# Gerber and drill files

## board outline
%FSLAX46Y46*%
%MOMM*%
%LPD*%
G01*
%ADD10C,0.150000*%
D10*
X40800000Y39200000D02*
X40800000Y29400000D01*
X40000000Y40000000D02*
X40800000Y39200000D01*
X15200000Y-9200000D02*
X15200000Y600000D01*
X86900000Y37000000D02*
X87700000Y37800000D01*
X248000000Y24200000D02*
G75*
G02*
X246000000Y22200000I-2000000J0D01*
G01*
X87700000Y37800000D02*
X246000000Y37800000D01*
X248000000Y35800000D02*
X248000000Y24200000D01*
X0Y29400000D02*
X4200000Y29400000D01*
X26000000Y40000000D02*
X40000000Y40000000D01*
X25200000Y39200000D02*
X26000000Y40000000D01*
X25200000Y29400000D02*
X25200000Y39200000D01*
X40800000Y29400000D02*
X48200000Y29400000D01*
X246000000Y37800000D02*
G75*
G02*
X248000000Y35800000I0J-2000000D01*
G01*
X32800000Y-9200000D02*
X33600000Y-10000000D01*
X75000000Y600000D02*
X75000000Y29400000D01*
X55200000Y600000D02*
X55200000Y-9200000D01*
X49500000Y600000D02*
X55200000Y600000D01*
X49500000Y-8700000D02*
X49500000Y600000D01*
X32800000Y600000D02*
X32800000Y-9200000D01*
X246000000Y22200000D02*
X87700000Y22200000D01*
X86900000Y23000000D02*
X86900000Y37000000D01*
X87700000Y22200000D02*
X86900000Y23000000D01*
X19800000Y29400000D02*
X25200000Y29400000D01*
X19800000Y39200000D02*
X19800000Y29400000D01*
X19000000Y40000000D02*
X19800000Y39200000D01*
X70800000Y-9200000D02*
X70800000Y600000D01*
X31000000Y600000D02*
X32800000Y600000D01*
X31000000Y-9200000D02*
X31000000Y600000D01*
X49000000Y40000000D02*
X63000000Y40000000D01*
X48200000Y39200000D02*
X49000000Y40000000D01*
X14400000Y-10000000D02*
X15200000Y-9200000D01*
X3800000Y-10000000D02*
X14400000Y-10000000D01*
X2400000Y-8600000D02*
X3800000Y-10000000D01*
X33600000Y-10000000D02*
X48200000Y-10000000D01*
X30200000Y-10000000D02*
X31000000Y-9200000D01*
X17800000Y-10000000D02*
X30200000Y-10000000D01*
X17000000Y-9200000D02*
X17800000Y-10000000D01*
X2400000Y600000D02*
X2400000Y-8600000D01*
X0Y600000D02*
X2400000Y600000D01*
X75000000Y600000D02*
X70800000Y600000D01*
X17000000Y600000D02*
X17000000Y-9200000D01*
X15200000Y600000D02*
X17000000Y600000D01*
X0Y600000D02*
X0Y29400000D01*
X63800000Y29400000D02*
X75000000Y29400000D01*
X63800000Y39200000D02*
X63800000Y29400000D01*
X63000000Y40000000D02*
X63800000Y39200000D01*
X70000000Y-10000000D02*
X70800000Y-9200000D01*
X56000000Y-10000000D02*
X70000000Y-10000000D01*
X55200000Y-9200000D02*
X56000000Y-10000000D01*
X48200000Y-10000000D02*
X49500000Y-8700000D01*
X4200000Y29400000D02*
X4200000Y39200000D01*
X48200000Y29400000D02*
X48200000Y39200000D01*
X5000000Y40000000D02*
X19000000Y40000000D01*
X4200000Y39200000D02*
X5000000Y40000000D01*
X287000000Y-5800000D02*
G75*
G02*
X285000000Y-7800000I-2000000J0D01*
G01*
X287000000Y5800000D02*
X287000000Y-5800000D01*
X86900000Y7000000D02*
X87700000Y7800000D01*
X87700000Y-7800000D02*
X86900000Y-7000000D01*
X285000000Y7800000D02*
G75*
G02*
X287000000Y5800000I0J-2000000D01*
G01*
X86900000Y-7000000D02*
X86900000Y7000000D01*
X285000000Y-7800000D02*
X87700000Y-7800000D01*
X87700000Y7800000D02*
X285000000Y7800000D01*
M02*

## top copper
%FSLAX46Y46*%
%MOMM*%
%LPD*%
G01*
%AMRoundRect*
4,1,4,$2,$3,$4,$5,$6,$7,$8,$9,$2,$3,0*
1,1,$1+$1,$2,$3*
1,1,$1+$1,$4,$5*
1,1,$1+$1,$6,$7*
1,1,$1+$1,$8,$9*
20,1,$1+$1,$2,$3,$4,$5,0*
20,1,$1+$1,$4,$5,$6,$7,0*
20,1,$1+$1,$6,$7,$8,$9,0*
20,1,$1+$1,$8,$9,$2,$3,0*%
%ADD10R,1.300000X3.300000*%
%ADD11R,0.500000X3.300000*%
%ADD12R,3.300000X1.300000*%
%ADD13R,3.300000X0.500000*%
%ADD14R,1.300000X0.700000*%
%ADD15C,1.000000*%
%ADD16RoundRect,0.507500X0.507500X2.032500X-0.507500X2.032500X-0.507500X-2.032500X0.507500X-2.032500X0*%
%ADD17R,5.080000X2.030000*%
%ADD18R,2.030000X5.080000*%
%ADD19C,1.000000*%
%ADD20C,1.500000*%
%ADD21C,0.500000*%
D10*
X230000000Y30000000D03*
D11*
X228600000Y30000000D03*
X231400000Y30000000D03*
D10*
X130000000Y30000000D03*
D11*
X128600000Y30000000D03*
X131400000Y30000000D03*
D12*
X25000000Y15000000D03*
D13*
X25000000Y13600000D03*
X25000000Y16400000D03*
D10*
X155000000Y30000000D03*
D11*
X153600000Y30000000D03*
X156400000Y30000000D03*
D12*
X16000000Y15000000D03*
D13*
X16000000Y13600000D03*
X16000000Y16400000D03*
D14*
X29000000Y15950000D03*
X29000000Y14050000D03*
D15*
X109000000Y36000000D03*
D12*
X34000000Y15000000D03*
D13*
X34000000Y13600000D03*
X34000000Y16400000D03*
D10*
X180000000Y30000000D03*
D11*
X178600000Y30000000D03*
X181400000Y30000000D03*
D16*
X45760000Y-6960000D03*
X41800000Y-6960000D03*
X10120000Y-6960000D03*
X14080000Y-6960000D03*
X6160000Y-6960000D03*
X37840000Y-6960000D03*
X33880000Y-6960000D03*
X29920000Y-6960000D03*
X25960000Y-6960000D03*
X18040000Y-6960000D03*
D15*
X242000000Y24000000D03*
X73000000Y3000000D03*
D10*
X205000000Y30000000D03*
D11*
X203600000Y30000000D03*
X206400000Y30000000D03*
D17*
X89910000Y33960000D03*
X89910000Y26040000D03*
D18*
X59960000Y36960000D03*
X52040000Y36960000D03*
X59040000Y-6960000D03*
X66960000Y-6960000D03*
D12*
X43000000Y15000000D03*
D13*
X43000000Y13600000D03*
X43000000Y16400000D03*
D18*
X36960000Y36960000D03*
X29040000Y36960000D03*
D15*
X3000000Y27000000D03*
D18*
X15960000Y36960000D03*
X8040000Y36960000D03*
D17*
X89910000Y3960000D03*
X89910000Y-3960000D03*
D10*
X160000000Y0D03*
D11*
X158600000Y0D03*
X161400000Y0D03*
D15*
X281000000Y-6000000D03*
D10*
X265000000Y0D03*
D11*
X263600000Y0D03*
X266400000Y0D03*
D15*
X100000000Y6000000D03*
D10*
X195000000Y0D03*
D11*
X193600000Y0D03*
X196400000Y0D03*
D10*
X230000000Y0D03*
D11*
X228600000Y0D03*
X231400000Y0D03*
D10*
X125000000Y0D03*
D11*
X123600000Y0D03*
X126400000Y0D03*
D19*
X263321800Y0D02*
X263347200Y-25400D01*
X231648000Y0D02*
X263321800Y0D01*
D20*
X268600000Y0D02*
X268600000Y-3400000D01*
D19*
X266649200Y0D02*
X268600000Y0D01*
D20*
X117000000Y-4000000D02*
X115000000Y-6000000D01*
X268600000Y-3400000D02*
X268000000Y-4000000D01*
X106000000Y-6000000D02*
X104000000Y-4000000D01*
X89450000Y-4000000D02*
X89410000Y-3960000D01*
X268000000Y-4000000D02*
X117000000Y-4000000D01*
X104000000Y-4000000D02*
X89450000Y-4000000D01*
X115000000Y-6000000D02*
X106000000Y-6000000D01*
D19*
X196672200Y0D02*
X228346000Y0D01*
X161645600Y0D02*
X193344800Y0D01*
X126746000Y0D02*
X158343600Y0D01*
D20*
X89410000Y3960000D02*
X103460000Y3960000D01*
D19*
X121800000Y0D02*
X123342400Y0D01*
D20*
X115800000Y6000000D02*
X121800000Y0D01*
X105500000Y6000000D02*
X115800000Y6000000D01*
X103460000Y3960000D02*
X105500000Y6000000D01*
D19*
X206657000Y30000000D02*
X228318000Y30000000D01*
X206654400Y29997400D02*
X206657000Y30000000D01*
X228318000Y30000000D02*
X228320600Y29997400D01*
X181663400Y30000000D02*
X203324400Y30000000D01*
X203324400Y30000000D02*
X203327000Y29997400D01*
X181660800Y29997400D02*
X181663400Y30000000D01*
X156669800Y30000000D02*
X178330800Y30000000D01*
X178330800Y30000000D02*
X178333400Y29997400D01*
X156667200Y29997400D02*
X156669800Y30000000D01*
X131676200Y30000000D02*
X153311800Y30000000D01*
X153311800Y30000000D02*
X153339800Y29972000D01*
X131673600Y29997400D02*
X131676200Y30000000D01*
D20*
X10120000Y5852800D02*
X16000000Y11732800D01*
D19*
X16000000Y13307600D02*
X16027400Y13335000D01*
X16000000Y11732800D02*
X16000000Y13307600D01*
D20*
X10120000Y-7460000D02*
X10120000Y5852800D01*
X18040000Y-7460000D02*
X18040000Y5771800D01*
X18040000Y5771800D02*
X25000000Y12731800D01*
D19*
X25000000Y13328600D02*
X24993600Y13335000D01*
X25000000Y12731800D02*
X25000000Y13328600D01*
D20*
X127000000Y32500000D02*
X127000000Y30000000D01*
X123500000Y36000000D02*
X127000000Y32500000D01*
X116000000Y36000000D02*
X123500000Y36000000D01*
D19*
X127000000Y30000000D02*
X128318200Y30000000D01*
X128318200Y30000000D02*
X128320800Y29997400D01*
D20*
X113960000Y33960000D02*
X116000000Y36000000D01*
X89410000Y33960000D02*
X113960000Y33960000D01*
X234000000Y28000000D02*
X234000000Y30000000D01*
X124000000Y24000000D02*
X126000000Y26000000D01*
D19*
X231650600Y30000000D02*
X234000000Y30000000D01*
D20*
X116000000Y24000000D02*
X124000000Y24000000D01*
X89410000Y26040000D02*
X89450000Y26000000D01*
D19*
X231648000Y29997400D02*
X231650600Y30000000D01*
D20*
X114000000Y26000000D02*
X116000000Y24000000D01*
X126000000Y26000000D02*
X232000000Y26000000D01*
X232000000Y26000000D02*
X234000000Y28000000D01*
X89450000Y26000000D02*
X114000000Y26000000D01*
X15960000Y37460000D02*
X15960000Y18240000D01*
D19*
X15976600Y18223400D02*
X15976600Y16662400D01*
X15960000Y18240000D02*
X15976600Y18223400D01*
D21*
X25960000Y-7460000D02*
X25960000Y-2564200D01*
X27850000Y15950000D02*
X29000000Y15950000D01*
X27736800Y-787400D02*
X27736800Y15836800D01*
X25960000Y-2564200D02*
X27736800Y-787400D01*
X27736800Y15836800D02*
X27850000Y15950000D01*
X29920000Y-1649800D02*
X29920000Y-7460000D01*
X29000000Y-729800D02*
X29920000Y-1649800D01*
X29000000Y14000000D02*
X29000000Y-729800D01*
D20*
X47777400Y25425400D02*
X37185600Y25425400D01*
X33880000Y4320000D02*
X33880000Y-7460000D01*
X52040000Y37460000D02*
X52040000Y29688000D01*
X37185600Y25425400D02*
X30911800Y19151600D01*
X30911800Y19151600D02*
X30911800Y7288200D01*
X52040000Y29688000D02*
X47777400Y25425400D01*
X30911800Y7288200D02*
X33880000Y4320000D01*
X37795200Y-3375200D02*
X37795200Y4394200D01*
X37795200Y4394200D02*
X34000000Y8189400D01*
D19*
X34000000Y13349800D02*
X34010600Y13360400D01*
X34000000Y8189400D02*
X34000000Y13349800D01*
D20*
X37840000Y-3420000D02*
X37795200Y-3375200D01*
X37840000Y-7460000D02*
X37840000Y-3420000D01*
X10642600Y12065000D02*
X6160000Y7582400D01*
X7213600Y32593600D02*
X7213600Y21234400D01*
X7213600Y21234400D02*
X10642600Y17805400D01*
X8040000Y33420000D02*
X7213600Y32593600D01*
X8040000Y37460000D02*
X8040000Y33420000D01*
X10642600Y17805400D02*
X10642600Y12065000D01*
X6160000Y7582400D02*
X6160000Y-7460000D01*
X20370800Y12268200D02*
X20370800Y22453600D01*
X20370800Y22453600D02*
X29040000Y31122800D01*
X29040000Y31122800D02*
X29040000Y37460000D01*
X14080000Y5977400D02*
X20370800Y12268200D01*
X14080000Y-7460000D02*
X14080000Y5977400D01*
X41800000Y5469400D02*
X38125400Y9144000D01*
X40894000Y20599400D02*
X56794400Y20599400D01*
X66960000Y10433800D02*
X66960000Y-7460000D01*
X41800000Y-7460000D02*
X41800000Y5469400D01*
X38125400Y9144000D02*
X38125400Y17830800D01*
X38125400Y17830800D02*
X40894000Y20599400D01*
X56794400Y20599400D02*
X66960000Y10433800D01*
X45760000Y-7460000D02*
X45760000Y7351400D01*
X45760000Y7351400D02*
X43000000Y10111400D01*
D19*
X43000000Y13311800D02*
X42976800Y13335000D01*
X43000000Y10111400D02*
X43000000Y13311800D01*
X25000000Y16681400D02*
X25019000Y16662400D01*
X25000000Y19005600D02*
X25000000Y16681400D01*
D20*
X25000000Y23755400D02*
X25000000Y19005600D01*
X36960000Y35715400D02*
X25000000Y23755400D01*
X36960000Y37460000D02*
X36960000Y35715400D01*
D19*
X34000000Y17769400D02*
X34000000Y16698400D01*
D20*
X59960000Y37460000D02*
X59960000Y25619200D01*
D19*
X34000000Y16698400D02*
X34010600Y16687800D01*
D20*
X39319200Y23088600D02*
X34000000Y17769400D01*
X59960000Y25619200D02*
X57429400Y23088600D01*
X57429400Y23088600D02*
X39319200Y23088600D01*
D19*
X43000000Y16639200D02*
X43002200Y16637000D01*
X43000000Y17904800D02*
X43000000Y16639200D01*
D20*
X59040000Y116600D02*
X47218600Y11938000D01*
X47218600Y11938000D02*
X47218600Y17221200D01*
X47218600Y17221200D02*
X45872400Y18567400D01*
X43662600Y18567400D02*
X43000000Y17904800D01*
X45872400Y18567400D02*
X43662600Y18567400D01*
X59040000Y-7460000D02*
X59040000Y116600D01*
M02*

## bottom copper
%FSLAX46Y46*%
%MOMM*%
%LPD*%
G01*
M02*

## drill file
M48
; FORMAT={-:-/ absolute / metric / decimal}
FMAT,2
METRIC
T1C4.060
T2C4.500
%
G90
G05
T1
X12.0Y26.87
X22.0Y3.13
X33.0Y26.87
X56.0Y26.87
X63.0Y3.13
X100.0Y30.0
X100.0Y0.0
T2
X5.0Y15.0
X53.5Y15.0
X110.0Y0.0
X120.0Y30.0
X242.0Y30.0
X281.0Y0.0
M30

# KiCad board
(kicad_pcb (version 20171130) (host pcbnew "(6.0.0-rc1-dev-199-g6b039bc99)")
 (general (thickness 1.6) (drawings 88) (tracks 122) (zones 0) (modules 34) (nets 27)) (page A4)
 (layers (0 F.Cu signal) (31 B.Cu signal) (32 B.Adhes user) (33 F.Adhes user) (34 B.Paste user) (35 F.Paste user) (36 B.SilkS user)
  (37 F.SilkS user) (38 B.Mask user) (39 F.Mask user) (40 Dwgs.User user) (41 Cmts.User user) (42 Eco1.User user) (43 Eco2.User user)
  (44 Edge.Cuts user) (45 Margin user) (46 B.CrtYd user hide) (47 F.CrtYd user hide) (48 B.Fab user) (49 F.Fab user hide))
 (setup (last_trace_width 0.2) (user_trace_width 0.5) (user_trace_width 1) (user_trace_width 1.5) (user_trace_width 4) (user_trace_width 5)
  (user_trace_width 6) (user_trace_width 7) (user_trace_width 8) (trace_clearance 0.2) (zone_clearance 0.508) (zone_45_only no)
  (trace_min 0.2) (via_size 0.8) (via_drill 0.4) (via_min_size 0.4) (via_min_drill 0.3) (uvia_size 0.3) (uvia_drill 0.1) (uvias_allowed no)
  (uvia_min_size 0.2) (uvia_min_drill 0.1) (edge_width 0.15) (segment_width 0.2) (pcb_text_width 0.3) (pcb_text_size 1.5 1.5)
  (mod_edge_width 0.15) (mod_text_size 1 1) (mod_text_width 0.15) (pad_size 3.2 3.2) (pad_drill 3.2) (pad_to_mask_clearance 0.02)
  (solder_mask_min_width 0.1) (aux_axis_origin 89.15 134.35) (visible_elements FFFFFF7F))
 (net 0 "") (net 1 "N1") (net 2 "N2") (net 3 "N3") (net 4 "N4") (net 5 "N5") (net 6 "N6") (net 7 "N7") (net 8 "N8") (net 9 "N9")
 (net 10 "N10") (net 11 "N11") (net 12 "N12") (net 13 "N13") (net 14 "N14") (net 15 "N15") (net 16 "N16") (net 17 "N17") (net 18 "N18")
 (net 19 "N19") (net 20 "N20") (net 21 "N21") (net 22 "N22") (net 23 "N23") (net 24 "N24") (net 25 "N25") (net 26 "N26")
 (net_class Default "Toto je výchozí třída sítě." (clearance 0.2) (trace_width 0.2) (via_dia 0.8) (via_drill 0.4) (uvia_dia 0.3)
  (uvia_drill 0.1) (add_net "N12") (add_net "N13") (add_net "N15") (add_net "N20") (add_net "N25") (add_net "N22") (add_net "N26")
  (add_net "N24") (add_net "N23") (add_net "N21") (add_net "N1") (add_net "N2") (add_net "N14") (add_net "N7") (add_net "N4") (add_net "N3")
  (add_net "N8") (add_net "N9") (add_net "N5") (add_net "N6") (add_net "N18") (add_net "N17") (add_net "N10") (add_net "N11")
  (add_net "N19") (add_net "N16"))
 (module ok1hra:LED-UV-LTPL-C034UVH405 (layer F.Cu) (at 230 -30)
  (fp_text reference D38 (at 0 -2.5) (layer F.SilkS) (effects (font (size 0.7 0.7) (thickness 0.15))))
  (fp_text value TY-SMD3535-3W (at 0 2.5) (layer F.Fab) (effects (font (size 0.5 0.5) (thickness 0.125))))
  (pad 3 smd rect (at 0 0) (size 1.3 3.3) (layers F.Cu F.Paste F.Mask))
  (pad 1 smd rect (at -1.4 0) (size 0.5 3.3) (layers F.Cu F.Paste F.Mask) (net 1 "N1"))
  (pad 2 smd rect (at 1.4 0) (size 0.5 3.3) (layers F.Cu F.Paste F.Mask) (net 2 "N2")))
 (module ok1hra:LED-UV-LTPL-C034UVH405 (layer F.Cu) (at 130 -30)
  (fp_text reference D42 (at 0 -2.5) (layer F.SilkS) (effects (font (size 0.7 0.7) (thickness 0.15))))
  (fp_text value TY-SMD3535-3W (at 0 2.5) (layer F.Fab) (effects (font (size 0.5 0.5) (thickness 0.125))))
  (pad 3 smd rect (at 0 0) (size 1.3 3.3) (layers F.Cu F.Paste F.Mask))
  (pad 1 smd rect (at -1.4 0) (size 0.5 3.3) (layers F.Cu F.Paste F.Mask) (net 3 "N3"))
  (pad 2 smd rect (at 1.4 0) (size 0.5 3.3) (layers F.Cu F.Paste F.Mask) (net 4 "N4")))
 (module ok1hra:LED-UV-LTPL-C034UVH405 (layer F.Cu) (at 25 -15 90)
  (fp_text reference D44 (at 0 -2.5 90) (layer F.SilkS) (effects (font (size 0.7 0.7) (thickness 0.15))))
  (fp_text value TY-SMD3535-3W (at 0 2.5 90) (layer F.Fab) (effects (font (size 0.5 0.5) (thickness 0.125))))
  (pad 3 smd rect (at 0 0 90) (size 1.3 3.3) (layers F.Cu F.Paste F.Mask))
  (pad 1 smd rect (at -1.4 0 90) (size 0.5 3.3) (layers F.Cu F.Paste F.Mask) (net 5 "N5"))
  (pad 2 smd rect (at 1.4 0 90) (size 0.5 3.3) (layers F.Cu F.Paste F.Mask) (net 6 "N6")))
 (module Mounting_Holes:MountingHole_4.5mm (layer F.Cu) (at 242 -30)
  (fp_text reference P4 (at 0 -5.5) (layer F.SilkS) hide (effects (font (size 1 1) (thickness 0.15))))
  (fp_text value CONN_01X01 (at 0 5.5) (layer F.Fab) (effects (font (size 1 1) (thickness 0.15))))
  (pad 1 np_thru_hole circle (at 0 0) (size 4.5 4.5) (drill 4.5) (layers *.Cu *.Mask)))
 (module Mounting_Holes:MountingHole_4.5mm (layer F.Cu) (at 5 -15)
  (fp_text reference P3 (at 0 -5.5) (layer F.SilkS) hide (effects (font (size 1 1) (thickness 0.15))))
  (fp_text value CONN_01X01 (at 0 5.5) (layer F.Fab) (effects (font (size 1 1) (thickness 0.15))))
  (pad 1 np_thru_hole circle (at 0 0) (size 4.5 4.5) (drill 4.5) (layers *.Cu *.Mask)))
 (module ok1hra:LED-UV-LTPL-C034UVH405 (layer F.Cu) (at 155 -30)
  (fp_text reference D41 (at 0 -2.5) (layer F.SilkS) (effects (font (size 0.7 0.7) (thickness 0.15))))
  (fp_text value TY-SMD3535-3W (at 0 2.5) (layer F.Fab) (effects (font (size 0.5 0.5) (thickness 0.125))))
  (pad 3 smd rect (at 0 0) (size 1.3 3.3) (layers F.Cu F.Paste F.Mask))
  (pad 1 smd rect (at -1.4 0) (size 0.5 3.3) (layers F.Cu F.Paste F.Mask) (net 4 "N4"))
  (pad 2 smd rect (at 1.4 0) (size 0.5 3.3) (layers F.Cu F.Paste F.Mask) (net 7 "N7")))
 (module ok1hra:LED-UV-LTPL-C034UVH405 (layer F.Cu) (at 16 -15 90)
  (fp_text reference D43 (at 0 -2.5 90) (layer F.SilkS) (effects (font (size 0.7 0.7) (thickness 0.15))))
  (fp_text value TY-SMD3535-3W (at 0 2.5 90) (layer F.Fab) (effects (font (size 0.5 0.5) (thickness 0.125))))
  (pad 3 smd rect (at 0 0 90) (size 1.3 3.3) (layers F.Cu F.Paste F.Mask))
  (pad 1 smd rect (at -1.4 0 90) (size 0.5 3.3) (layers F.Cu F.Paste F.Mask) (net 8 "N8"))
  (pad 2 smd rect (at 1.4 0 90) (size 0.5 3.3) (layers F.Cu F.Paste F.Mask) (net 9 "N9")))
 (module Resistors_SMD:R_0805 (layer F.Cu) (at 29 -15 270)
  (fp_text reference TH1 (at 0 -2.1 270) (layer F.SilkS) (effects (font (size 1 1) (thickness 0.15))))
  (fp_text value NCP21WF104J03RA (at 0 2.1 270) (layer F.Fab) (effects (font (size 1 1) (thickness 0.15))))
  (pad 1 smd rect (at -0.95 0 270) (size 0.7 1.3) (layers F.Cu F.Paste F.Mask) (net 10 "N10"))
  (pad 2 smd rect (at 0.95 0 270) (size 0.7 1.3) (layers F.Cu F.Paste F.Mask) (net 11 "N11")))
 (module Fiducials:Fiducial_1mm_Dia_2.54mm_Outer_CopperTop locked (layer F.Cu) (at 109 -36)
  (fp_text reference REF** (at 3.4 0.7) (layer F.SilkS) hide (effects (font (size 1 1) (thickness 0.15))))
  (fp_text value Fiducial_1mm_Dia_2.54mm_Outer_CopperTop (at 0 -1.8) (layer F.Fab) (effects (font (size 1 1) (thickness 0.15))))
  (pad ~ smd circle (at 0 0) (size 1 1) (layers F.Cu F.Mask) (solder_mask_margin 0.77) (clearance 0.77)))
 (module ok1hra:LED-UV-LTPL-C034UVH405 (layer F.Cu) (at 34 -15 90)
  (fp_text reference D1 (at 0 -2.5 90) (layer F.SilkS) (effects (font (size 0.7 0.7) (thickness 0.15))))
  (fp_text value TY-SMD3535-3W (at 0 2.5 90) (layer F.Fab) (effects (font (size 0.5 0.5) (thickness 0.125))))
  (pad 3 smd rect (at 0 0 90) (size 1.3 3.3) (layers F.Cu F.Paste F.Mask))
  (pad 1 smd rect (at -1.4 0 90) (size 0.5 3.3) (layers F.Cu F.Paste F.Mask) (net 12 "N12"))
  (pad 2 smd rect (at 1.4 0 90) (size 0.5 3.3) (layers F.Cu F.Paste F.Mask) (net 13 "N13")))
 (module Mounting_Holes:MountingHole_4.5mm (layer F.Cu) (at 53.5 -15)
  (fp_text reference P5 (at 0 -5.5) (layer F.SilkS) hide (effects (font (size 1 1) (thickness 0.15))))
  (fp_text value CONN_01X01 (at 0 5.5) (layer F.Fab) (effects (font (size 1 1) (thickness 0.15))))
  (pad 1 np_thru_hole circle (at 0 0) (size 4.5 4.5) (drill 4.5) (layers *.Cu *.Mask)))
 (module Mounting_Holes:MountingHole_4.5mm (layer F.Cu) (at 120 -30)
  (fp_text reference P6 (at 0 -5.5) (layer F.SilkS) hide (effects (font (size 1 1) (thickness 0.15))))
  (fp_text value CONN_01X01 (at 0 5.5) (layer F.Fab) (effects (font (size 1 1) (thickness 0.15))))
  (pad 1 np_thru_hole circle (at 0 0) (size 4.5 4.5) (drill 4.5) (layers *.Cu *.Mask)))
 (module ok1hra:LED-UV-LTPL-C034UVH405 (layer F.Cu) (at 180 -30)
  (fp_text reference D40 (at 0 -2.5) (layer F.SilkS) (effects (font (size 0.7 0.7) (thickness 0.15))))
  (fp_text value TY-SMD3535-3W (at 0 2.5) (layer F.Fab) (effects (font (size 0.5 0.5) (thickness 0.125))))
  (pad 3 smd rect (at 0 0) (size 1.3 3.3) (layers F.Cu F.Paste F.Mask))
  (pad 1 smd rect (at -1.4 0) (size 0.5 3.3) (layers F.Cu F.Paste F.Mask) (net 7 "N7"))
  (pad 2 smd rect (at 1.4 0) (size 0.5 3.3) (layers F.Cu F.Paste F.Mask) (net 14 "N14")))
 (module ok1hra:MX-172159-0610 (layer F.Cu) (at 22 10 180)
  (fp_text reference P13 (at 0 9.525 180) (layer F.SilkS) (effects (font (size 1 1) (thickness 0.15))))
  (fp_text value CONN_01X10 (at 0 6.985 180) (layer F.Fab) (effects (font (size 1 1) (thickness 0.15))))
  (pad 10 smd roundrect (at -23.76 3.04 180) (size 2.03 5.08) (layers F.Cu F.Mask) (roundrect_rratio 0.25) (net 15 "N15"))
  (pad 9 smd roundrect (at -19.8 3.04 180) (size 2.03 5.08) (layers F.Cu F.Mask) (roundrect_rratio 0.25) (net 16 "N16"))
  (pad 2 smd roundrect (at 11.88 3.04 180) (size 2.03 5.08) (layers F.Cu F.Mask) (roundrect_rratio 0.25) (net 8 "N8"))
  (pad 3 smd roundrect (at 7.92 3.04 180) (size 2.03 5.08) (layers F.Cu F.Mask) (roundrect_rratio 0.25) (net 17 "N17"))
  (pad 1 smd roundrect (at 15.84 3.04 180) (size 2.03 5.08) (layers F.Cu F.Mask) (roundrect_rratio 0.25) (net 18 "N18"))
  (pad 8 smd roundrect (at -15.84 3.04 180) (size 2.03 5.08) (layers F.Cu F.Mask) (roundrect_rratio 0.25) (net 12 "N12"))
  (pad 7 smd roundrect (at -11.88 3.04 180) (size 2.03 5.08) (layers F.Cu F.Mask) (roundrect_rratio 0.25) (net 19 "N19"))
  (pad 6 smd roundrect (at -7.92 3.04 180) (size 2.03 5.08) (layers F.Cu F.Mask) (roundrect_rratio 0.25) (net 11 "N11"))
  (pad 5 smd roundrect (at -3.96 3.04 180) (size 2.03 5.08) (layers F.Cu F.Mask) (roundrect_rratio 0.25) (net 10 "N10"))
  (pad 4 smd roundrect (at 3.96 3.04 180) (size 2.03 5.08) (layers F.Cu F.Mask) (roundrect_rratio 0.25) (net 5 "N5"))
  (pad "" np_thru_hole circle (at 0 13.13 180) (size 4.06 4.06) (drill 4.06) (layers *.Cu *.Mask)))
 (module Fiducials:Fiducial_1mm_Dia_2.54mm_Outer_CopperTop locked (layer F.Cu) (at 242 -24)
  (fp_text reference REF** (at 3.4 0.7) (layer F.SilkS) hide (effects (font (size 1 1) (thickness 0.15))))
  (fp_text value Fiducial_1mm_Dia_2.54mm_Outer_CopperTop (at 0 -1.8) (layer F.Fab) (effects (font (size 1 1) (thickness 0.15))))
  (pad ~ smd circle (at 0 0) (size 1 1) (layers F.Cu F.Mask) (solder_mask_margin 0.77) (clearance 0.77)))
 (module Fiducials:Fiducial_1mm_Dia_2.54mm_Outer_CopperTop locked (layer F.Cu) (at 73 -3)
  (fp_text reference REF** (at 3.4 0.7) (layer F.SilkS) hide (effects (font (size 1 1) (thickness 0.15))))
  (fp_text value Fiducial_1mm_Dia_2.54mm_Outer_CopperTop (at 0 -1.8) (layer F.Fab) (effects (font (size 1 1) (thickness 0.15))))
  (pad ~ smd circle (at 0 0) (size 1 1) (layers F.Cu F.Mask) (solder_mask_margin 0.77) (clearance 0.77)))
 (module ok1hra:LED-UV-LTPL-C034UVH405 (layer F.Cu) (at 205 -30)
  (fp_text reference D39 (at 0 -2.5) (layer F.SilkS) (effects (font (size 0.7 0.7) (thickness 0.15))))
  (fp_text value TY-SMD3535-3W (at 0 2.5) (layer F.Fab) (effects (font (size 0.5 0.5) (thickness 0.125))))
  (pad 3 smd rect (at 0 0) (size 1.3 3.3) (layers F.Cu F.Paste F.Mask))
  (pad 1 smd rect (at -1.4 0) (size 0.5 3.3) (layers F.Cu F.Paste F.Mask) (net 14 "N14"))
  (pad 2 smd rect (at 1.4 0) (size 0.5 3.3) (layers F.Cu F.Paste F.Mask) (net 1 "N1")))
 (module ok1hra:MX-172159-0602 (layer F.Cu) (at 86.87 -30 90)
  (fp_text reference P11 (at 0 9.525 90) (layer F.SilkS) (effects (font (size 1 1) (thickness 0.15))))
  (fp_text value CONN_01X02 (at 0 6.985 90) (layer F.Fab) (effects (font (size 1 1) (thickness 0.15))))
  (pad "" np_thru_hole circle (at 0 13.13 90) (size 4.06 4.06) (drill 4.06) (layers *.Cu *.Mask))
  (pad 1 smd rect (at 3.96 3.04 90) (size 2.03 5.08) (layers F.Cu F.Mask) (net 3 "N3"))
  (pad 2 smd rect (at -3.96 3.04 90) (size 2.03 5.08) (layers F.Cu F.Mask) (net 2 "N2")))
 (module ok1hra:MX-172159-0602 (layer F.Cu) (at 56 -40)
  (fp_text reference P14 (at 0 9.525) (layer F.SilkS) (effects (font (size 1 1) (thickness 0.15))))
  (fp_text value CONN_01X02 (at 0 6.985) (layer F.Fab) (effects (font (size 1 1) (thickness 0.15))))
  (pad "" np_thru_hole circle (at 0 13.13) (size 4.06 4.06) (drill 4.06) (layers *.Cu *.Mask))
  (pad 1 smd rect (at 3.96 3.04) (size 2.03 5.08) (layers F.Cu F.Mask) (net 13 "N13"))
  (pad 2 smd rect (at -3.96 3.04) (size 2.03 5.08) (layers F.Cu F.Mask) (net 19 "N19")))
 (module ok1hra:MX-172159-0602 (layer F.Cu) (at 63 10 180)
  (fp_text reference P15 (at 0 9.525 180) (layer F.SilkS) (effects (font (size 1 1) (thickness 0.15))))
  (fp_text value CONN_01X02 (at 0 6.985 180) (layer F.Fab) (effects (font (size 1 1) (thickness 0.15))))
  (pad "" np_thru_hole circle (at 0 13.13 180) (size 4.06 4.06) (drill 4.06) (layers *.Cu *.Mask))
  (pad 1 smd rect (at 3.96 3.04 180) (size 2.03 5.08) (layers F.Cu F.Mask) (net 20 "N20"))
  (pad 2 smd rect (at -3.96 3.04 180) (size 2.03 5.08) (layers F.Cu F.Mask) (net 16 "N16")))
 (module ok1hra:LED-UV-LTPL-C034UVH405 (layer F.Cu) (at 43 -15 90)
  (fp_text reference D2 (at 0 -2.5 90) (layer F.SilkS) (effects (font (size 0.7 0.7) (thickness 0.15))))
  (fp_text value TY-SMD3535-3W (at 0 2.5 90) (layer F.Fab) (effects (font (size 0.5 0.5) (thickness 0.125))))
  (pad 3 smd rect (at 0 0 90) (size 1.3 3.3) (layers F.Cu F.Paste F.Mask))
  (pad 1 smd rect (at -1.4 0 90) (size 0.5 3.3) (layers F.Cu F.Paste F.Mask) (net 15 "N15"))
  (pad 2 smd rect (at 1.4 0 90) (size 0.5 3.3) (layers F.Cu F.Paste F.Mask) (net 20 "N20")))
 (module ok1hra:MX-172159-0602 (layer F.Cu) (at 33 -40)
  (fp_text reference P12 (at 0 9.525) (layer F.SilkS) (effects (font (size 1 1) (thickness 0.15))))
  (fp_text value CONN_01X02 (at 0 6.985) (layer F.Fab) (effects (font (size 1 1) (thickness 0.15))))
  (pad "" np_thru_hole circle (at 0 13.13) (size 4.06 4.06) (drill 4.06) (layers *.Cu *.Mask))
  (pad 1 smd rect (at 3.96 3.04) (size 2.03 5.08) (layers F.Cu F.Mask) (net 6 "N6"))
  (pad 2 smd rect (at -3.96 3.04) (size 2.03 5.08) (layers F.Cu F.Mask) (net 17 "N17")))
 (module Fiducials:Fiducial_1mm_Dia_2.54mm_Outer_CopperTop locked (layer F.Cu) (at 3 -27)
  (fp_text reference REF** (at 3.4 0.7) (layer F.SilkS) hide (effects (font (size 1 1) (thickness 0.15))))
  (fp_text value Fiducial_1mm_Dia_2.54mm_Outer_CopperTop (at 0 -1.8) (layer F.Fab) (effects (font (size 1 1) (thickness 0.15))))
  (pad ~ smd circle (at 0 0) (size 1 1) (layers F.Cu F.Mask) (solder_mask_margin 0.77) (clearance 0.77)))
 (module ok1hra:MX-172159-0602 (layer F.Cu) (at 12 -40)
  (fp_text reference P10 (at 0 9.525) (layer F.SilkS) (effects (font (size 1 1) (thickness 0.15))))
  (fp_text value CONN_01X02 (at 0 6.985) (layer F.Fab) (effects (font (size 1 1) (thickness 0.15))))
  (pad "" np_thru_hole circle (at 0 13.13) (size 4.06 4.06) (drill 4.06) (layers *.Cu *.Mask))
  (pad 1 smd rect (at 3.96 3.04) (size 2.03 5.08) (layers F.Cu F.Mask) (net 9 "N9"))
  (pad 2 smd rect (at -3.96 3.04) (size 2.03 5.08) (layers F.Cu F.Mask) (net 18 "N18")))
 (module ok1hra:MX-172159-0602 (layer F.Cu) (at 86.87 0 90)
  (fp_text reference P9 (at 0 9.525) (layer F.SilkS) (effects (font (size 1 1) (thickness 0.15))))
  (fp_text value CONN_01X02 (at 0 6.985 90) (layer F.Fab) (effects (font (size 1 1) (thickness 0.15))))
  (pad "" np_thru_hole circle (at 0 13.13 90) (size 4.06 4.06) (drill 4.06) (layers *.Cu *.Mask))
  (pad 1 smd rect (at 3.96 3.04 90) (size 2.03 5.08) (layers F.Cu F.Mask) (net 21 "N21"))
  (pad 2 smd rect (at -3.96 3.04 90) (size 2.03 5.08) (layers F.Cu F.Mask) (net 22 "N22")))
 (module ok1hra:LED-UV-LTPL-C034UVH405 (layer F.Cu) (at 160 0)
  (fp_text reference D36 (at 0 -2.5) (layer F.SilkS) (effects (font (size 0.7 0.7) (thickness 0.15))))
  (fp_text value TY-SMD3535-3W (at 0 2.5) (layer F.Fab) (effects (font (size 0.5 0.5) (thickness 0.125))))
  (pad 3 smd rect (at 0 0) (size 1.3 3.3) (layers F.Cu F.Paste F.Mask))
  (pad 1 smd rect (at -1.4 0) (size 0.5 3.3) (layers F.Cu F.Paste F.Mask) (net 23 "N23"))
  (pad 2 smd rect (at 1.4 0) (size 0.5 3.3) (layers F.Cu F.Paste F.Mask) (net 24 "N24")))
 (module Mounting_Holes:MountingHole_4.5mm (layer F.Cu) (at 281 0)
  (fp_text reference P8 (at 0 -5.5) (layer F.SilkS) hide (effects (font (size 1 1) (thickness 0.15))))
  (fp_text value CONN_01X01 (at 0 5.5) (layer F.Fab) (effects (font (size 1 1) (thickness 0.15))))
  (pad 1 np_thru_hole circle (at 0 0) (size 4.5 4.5) (drill 4.5) (layers *.Cu *.Mask)))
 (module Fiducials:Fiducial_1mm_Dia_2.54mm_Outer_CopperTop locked (layer F.Cu) (at 281 6)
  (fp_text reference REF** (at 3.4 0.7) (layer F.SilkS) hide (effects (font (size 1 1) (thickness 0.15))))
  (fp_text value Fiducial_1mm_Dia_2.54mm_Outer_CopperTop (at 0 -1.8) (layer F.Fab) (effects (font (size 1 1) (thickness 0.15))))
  (pad ~ smd circle (at 0 0) (size 1 1) (layers F.Cu F.Mask) (solder_mask_margin 0.77) (clearance 0.77)))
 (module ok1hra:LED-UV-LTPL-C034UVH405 (layer F.Cu) (at 265 0)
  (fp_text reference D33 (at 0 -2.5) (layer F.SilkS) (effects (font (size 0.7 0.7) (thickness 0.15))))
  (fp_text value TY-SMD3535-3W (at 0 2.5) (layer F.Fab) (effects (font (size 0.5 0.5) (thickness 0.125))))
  (pad 3 smd rect (at 0 0) (size 1.3 3.3) (layers F.Cu F.Paste F.Mask))
  (pad 1 smd rect (at -1.4 0) (size 0.5 3.3) (layers F.Cu F.Paste F.Mask) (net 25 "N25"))
  (pad 2 smd rect (at 1.4 0) (size 0.5 3.3) (layers F.Cu F.Paste F.Mask) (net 22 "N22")))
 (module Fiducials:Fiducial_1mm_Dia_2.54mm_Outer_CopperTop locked (layer F.Cu) (at 100 -6)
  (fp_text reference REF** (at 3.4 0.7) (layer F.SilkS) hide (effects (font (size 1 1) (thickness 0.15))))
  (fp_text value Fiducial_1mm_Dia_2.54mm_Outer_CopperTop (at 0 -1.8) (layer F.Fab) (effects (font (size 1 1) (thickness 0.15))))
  (pad ~ smd circle (at 0 0) (size 1 1) (layers F.Cu F.Mask) (solder_mask_margin 0.77) (clearance 0.77)))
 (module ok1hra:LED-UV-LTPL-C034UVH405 (layer F.Cu) (at 195 0)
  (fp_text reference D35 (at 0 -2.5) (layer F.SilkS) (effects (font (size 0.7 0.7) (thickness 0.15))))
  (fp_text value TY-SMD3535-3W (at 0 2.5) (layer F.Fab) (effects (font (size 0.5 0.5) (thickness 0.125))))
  (pad 3 smd rect (at 0 0) (size 1.3 3.3) (layers F.Cu F.Paste F.Mask))
  (pad 1 smd rect (at -1.4 0) (size 0.5 3.3) (layers F.Cu F.Paste F.Mask) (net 24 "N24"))
  (pad 2 smd rect (at 1.4 0) (size 0.5 3.3) (layers F.Cu F.Paste F.Mask) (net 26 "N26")))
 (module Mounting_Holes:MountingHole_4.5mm (layer F.Cu) (at 110 0)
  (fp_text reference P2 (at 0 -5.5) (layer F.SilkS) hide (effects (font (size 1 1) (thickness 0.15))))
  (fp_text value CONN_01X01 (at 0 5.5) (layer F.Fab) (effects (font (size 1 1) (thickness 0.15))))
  (pad 1 np_thru_hole circle (at 0 0) (size 4.5 4.5) (drill 4.5) (layers *.Cu *.Mask)))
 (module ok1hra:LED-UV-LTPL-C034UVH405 (layer F.Cu) (at 230 0)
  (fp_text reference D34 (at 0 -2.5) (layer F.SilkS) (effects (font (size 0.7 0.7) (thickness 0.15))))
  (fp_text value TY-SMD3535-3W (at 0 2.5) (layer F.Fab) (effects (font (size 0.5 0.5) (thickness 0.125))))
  (pad 3 smd rect (at 0 0) (size 1.3 3.3) (layers F.Cu F.Paste F.Mask))
  (pad 1 smd rect (at -1.4 0) (size 0.5 3.3) (layers F.Cu F.Paste F.Mask) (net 26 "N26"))
  (pad 2 smd rect (at 1.4 0) (size 0.5 3.3) (layers F.Cu F.Paste F.Mask) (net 25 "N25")))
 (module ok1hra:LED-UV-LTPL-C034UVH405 (layer F.Cu) (at 125 0)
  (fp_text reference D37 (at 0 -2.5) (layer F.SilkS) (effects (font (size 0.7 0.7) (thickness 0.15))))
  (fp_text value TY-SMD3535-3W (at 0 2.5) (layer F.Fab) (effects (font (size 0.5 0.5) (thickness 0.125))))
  (pad 3 smd rect (at 0 0) (size 1.3 3.3) (layers F.Cu F.Paste F.Mask))
  (pad 1 smd rect (at -1.4 0) (size 0.5 3.3) (layers F.Cu F.Paste F.Mask) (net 21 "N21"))
  (pad 2 smd rect (at 1.4 0) (size 0.5 3.3) (layers F.Cu F.Paste F.Mask) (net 23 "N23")))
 (gr_line (start 40.8 -39.2) (end 40.8 -29.4) (layer Edge.Cuts) (width 0.15))
 (gr_line (start 40 -40) (end 40.8 -39.2) (layer Edge.Cuts) (width 0.15))
 (gr_line (start 15.2 9.2) (end 15.2 -0.6) (layer Edge.Cuts) (width 0.15))
 (gr_line (start 86.9 -37) (end 87.7 -37.8) (layer Edge.Cuts) (width 0.15))
 (gr_arc (start 246 -24.2) (end 246 -22.2) (angle -90) (layer Edge.Cuts) (width 0.15))
 (gr_line (start 87.7 -37.8) (end 246 -37.8) (layer Edge.Cuts) (width 0.15))
 (gr_line (start 248 -35.8) (end 248 -24.2) (layer Edge.Cuts) (width 0.15))
 (gr_line (start 0 -29.4) (end 4.2 -29.4) (layer Edge.Cuts) (width 0.15))
 (gr_line (start 26 -40) (end 40 -40) (layer Edge.Cuts) (width 0.15))
 (gr_line (start 25.2 -39.2) (end 26 -40) (layer Edge.Cuts) (width 0.15))
 (gr_line (start 25.2 -29.4) (end 25.2 -39.2) (layer Edge.Cuts) (width 0.15))
 (gr_line (start 40.8 -29.4) (end 48.2 -29.4) (layer Edge.Cuts) (width 0.15))
 (gr_arc (start 246 -35.8) (end 248 -35.8) (angle -90) (layer Edge.Cuts) (width 0.15))
 (gr_line (start 32.8 9.2) (end 33.6 10) (layer Edge.Cuts) (width 0.15))
 (gr_line (start 75 -0.6) (end 75 -29.4) (layer Edge.Cuts) (width 0.15))
 (gr_line (start 55.2 -0.6) (end 55.2 9.2) (layer Edge.Cuts) (width 0.15))
 (gr_line (start 49.5 -0.6) (end 55.2 -0.6) (layer Edge.Cuts) (width 0.15))
 (gr_line (start 49.5 8.7) (end 49.5 -0.6) (layer Edge.Cuts) (width 0.15))
 (gr_line (start 32.8 -0.6) (end 32.8 9.2) (layer Edge.Cuts) (width 0.15))
 (gr_line (start 246 -22.2) (end 87.7 -22.2) (layer Edge.Cuts) (width 0.15))
 (gr_line (start 86.9 -23) (end 86.9 -37) (layer Edge.Cuts) (width 0.15))
 (gr_line (start 87.7 -22.2) (end 86.9 -23) (layer Edge.Cuts) (width 0.15))
 (gr_line (start 19.8 -29.4) (end 25.2 -29.4) (layer Edge.Cuts) (width 0.15))
 (gr_line (start 19.8 -39.2) (end 19.8 -29.4) (layer Edge.Cuts) (width 0.15))
 (gr_line (start 19 -40) (end 19.8 -39.2) (layer Edge.Cuts) (width 0.15))
 (gr_line (start 70.8 9.2) (end 70.8 -0.6) (layer Edge.Cuts) (width 0.15))
 (gr_line (start 31 -0.6) (end 32.8 -0.6) (layer Edge.Cuts) (width 0.15))
 (gr_line (start 31 9.2) (end 31 -0.6) (layer Edge.Cuts) (width 0.15))
 (gr_line (start 49 -40) (end 63 -40) (layer Edge.Cuts) (width 0.15))
 (gr_line (start 48.2 -39.2) (end 49 -40) (layer Edge.Cuts) (width 0.15))
 (gr_line (start 14.4 10) (end 15.2 9.2) (layer Edge.Cuts) (width 0.15))
 (gr_line (start 3.8 10) (end 14.4 10) (layer Edge.Cuts) (width 0.15))
 (gr_line (start 2.4 8.6) (end 3.8 10) (layer Edge.Cuts) (width 0.15))
 (gr_line (start 33.6 10) (end 48.2 10) (layer Edge.Cuts) (width 0.15))
 (gr_line (start 30.2 10) (end 31 9.2) (layer Edge.Cuts) (width 0.15))
 (gr_line (start 17.8 10) (end 30.2 10) (layer Edge.Cuts) (width 0.15))
 (gr_line (start 17 9.2) (end 17.8 10) (layer Edge.Cuts) (width 0.15))
 (gr_line (start 2.4 -0.6) (end 2.4 8.6) (layer Edge.Cuts) (width 0.15))
 (gr_line (start 0 -0.6) (end 2.4 -0.6) (layer Edge.Cuts) (width 0.15))
 (gr_line (start 75 -0.6) (end 70.8 -0.6) (layer Edge.Cuts) (width 0.15))
 (gr_line (start 17 -0.6) (end 17 9.2) (layer Edge.Cuts) (width 0.15))
 (gr_line (start 15.2 -0.6) (end 17 -0.6) (layer Edge.Cuts) (width 0.15))
 (gr_line (start 0 -0.6) (end 0 -29.4) (layer Edge.Cuts) (width 0.15))
 (gr_line (start 63.8 -29.4) (end 75 -29.4) (layer Edge.Cuts) (width 0.15))
 (gr_line (start 63.8 -39.2) (end 63.8 -29.4) (layer Edge.Cuts) (width 0.15))
 (gr_line (start 63 -40) (end 63.8 -39.2) (layer Edge.Cuts) (width 0.15))
 (gr_line (start 70 10) (end 70.8 9.2) (layer Edge.Cuts) (width 0.15))
 (gr_line (start 56 10) (end 70 10) (layer Edge.Cuts) (width 0.15))
 (gr_line (start 55.2 9.2) (end 56 10) (layer Edge.Cuts) (width 0.15))
 (gr_line (start 48.2 10) (end 49.5 8.7) (layer Edge.Cuts) (width 0.15))
 (gr_line (start 4.2 -29.4) (end 4.2 -39.2) (layer Edge.Cuts) (width 0.15))
 (gr_line (start 48.2 -29.4) (end 48.2 -39.2) (layer Edge.Cuts) (width 0.15))
 (gr_line (start 5 -40) (end 19 -40) (layer Edge.Cuts) (width 0.15))
 (gr_line (start 4.2 -39.2) (end 5 -40) (layer Edge.Cuts) (width 0.15))
 (gr_arc (start 285 5.8) (end 285 7.8) (angle -90) (layer Edge.Cuts) (width 0.15))
 (gr_line (start 287 -5.8) (end 287 5.8) (layer Edge.Cuts) (width 0.15))
 (gr_line (start 86.9 -7) (end 87.7 -7.8) (layer Edge.Cuts) (width 0.15))
 (gr_line (start 87.7 7.8) (end 86.9 7) (layer Edge.Cuts) (width 0.15))
 (gr_arc (start 285 -5.8) (end 287 -5.8) (angle -90) (layer Edge.Cuts) (width 0.15))
 (gr_line (start 86.9 7) (end 86.9 -7) (layer Edge.Cuts) (width 0.15))
 (gr_line (start 285 7.8) (end 87.7 7.8) (layer Edge.Cuts) (width 0.15))
 (gr_line (start 87.7 -7.8) (end 285 -7.8) (layer Edge.Cuts) (width 0.15))
 (segment (start 263.3218 0) (end 263.3472 0.0254) (width 1) (layer F.Cu) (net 25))
 (segment (start 231.648 0) (end 263.3218 0) (width 1) (layer F.Cu) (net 25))
 (segment (start 268.6 0) (end 268.6 3.4) (width 1.5) (layer F.Cu) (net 22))
 (segment (start 266.6492 0) (end 268.6 0) (width 1) (layer F.Cu) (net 22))
 (segment (start 117 4) (end 115 6) (width 1.5) (layer F.Cu) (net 22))
 (segment (start 268.6 3.4) (end 268 4) (width 1.5) (layer F.Cu) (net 22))
 (segment (start 106 6) (end 104 4) (width 1.5) (layer F.Cu) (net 22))
 (segment (start 89.45 4) (end 89.41 3.96) (width 1.5) (layer F.Cu) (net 22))
 (segment (start 268 4) (end 117 4) (width 1.5) (layer F.Cu) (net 22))
 (segment (start 104 4) (end 89.45 4) (width 1.5) (layer F.Cu) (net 22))
 (segment (start 115 6) (end 106 6) (width 1.5) (layer F.Cu) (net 22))
 (segment (start 196.6722 0) (end 228.346 0) (width 1) (layer F.Cu) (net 26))
 (segment (start 161.6456 0) (end 193.3448 0) (width 1) (layer F.Cu) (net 24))
 (segment (start 126.746 0) (end 158.3436 0) (width 1) (layer F.Cu) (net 23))
 (segment (start 89.41 -3.96) (end 103.46 -3.96) (width 1.5) (layer F.Cu) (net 21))
 (segment (start 121.8 0) (end 123.3424 0) (width 1) (layer F.Cu) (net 21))
 (segment (start 115.8 -6) (end 121.8 0) (width 1.5) (layer F.Cu) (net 21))
 (segment (start 105.5 -6) (end 115.8 -6) (width 1.5) (layer F.Cu) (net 21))
 (segment (start 103.46 -3.96) (end 105.5 -6) (width 1.5) (layer F.Cu) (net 21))
 (segment (start 206.657 -30) (end 228.318 -30) (width 1) (layer F.Cu) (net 1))
 (segment (start 206.6544 -29.9974) (end 206.657 -30) (width 1) (layer F.Cu) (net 1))
 (segment (start 228.318 -30) (end 228.3206 -29.9974) (width 1) (layer F.Cu) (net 1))
 (segment (start 181.6634 -30) (end 203.3244 -30) (width 1) (layer F.Cu) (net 14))
 (segment (start 203.3244 -30) (end 203.327 -29.9974) (width 1) (layer F.Cu) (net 14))
 (segment (start 181.6608 -29.9974) (end 181.6634 -30) (width 1) (layer F.Cu) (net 14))
 (segment (start 156.6698 -30) (end 178.3308 -30) (width 1) (layer F.Cu) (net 7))
 (segment (start 178.3308 -30) (end 178.3334 -29.9974) (width 1) (layer F.Cu) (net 7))
 (segment (start 156.6672 -29.9974) (end 156.6698 -30) (width 1) (layer F.Cu) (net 7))
 (segment (start 131.6762 -30) (end 153.3118 -30) (width 1) (layer F.Cu) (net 4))
 (segment (start 153.3118 -30) (end 153.3398 -29.972) (width 1) (layer F.Cu) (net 4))
 (segment (start 131.6736 -29.9974) (end 131.6762 -30) (width 1) (layer F.Cu) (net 4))
 (segment (start 10.12 -5.8528) (end 16 -11.7328) (width 1.5) (layer F.Cu) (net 8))
 (segment (start 16 -13.3076) (end 16.0274 -13.335) (width 1) (layer F.Cu) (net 8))
 (segment (start 16 -11.7328) (end 16 -13.3076) (width 1) (layer F.Cu) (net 8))
 (segment (start 10.12 7.46) (end 10.12 -5.8528) (width 1.5) (layer F.Cu) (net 8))
 (segment (start 18.04 7.46) (end 18.04 -5.7718) (width 1.5) (layer F.Cu) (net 5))
 (segment (start 18.04 -5.7718) (end 25 -12.7318) (width 1.5) (layer F.Cu) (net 5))
 (segment (start 25 -13.3286) (end 24.9936 -13.335) (width 1) (layer F.Cu) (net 5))
 (segment (start 25 -12.7318) (end 25 -13.3286) (width 1) (layer F.Cu) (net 5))
 (segment (start 127 -32.5) (end 127 -30) (width 1.5) (layer F.Cu) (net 3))
 (segment (start 123.5 -36) (end 127 -32.5) (width 1.5) (layer F.Cu) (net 3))
 (segment (start 116 -36) (end 123.5 -36) (width 1.5) (layer F.Cu) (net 3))
 (segment (start 127 -30) (end 128.3182 -30) (width 1) (layer F.Cu) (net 3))
 (segment (start 128.3182 -30) (end 128.3208 -29.9974) (width 1) (layer F.Cu) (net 3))
 (segment (start 113.96 -33.96) (end 116 -36) (width 1.5) (layer F.Cu) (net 3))
 (segment (start 89.41 -33.96) (end 113.96 -33.96) (width 1.5) (layer F.Cu) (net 3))
 (segment (start 234 -28) (end 234 -30) (width 1.5) (layer F.Cu) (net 2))
 (segment (start 124 -24) (end 126 -26) (width 1.5) (layer F.Cu) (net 2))
 (segment (start 231.6506 -30) (end 234 -30) (width 1) (layer F.Cu) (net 2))
 (segment (start 116 -24) (end 124 -24) (width 1.5) (layer F.Cu) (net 2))
 (segment (start 89.41 -26.04) (end 89.45 -26) (width 1.5) (layer F.Cu) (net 2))
 (segment (start 231.648 -29.9974) (end 231.6506 -30) (width 1) (layer F.Cu) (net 2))
 (segment (start 114 -26) (end 116 -24) (width 1.5) (layer F.Cu) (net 2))
 (segment (start 126 -26) (end 232 -26) (width 1.5) (layer F.Cu) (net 2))
 (segment (start 232 -26) (end 234 -28) (width 1.5) (layer F.Cu) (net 2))
 (segment (start 89.45 -26) (end 114 -26) (width 1.5) (layer F.Cu) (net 2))
 (segment (start 15.96 -37.46) (end 15.96 -18.24) (width 1.5) (layer F.Cu) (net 9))
 (segment (start 15.9766 -18.2234) (end 15.9766 -16.6624) (width 1) (layer F.Cu) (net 9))
 (segment (start 15.96 -18.24) (end 15.9766 -18.2234) (width 1) (layer F.Cu) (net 9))
 (segment (start 25.96 7.46) (end 25.96 2.5642) (width 0.5) (layer F.Cu) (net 10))
 (segment (start 27.85 -15.95) (end 29 -15.95) (width 0.5) (layer F.Cu) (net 10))
 (segment (start 27.7368 0.7874) (end 27.7368 -15.8368) (width 0.5) (layer F.Cu) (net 10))
 (segment (start 25.96 2.5642) (end 27.7368 0.7874) (width 0.5) (layer F.Cu) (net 10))
 (segment (start 27.7368 -15.8368) (end 27.85 -15.95) (width 0.5) (layer F.Cu) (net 10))
 (segment (start 29.92 1.6498) (end 29.92 7.46) (width 0.5) (layer F.Cu) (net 11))
 (segment (start 29 0.7298) (end 29.92 1.6498) (width 0.5) (layer F.Cu) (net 11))
 (segment (start 29 -14) (end 29 0.7298) (width 0.5) (layer F.Cu) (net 11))
 (segment (start 47.7774 -25.4254) (end 37.1856 -25.4254) (width 1.5) (layer F.Cu) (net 19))
 (segment (start 33.88 -4.32) (end 33.88 7.46) (width 1.5) (layer F.Cu) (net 19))
 (segment (start 52.04 -37.46) (end 52.04 -29.688) (width 1.5) (layer F.Cu) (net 19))
 (segment (start 37.1856 -25.4254) (end 30.9118 -19.1516) (width 1.5) (layer F.Cu) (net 19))
 (segment (start 30.9118 -19.1516) (end 30.9118 -7.2882) (width 1.5) (layer F.Cu) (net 19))
 (segment (start 52.04 -29.688) (end 47.7774 -25.4254) (width 1.5) (layer F.Cu) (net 19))
 (segment (start 30.9118 -7.2882) (end 33.88 -4.32) (width 1.5) (layer F.Cu) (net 19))
 (segment (start 37.7952 3.3752) (end 37.7952 -4.3942) (width 1.5) (layer F.Cu) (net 12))
 (segment (start 37.7952 -4.3942) (end 34 -8.1894) (width 1.5) (layer F.Cu) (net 12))
 (segment (start 34 -13.3498) (end 34.0106 -13.3604) (width 1) (layer F.Cu) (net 12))
 (segment (start 34 -8.1894) (end 34 -13.3498) (width 1) (layer F.Cu) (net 12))
 (segment (start 37.84 3.42) (end 37.7952 3.3752) (width 1.5) (layer F.Cu) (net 12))
 (segment (start 37.84 7.46) (end 37.84 3.42) (width 1.5) (layer F.Cu) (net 12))
 (segment (start 10.6426 -12.065) (end 6.16 -7.5824) (width 1.5) (layer F.Cu) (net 18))
 (segment (start 7.2136 -32.5936) (end 7.2136 -21.2344) (width 1.5) (layer F.Cu) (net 18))
 (segment (start 7.2136 -21.2344) (end 10.6426 -17.8054) (width 1.5) (layer F.Cu) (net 18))
 (segment (start 8.04 -33.42) (end 7.2136 -32.5936) (width 1.5) (layer F.Cu) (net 18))
 (segment (start 8.04 -37.46) (end 8.04 -33.42) (width 1.5) (layer F.Cu) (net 18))
 (segment (start 10.6426 -17.8054) (end 10.6426 -12.065) (width 1.5) (layer F.Cu) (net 18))
 (segment (start 6.16 -7.5824) (end 6.16 7.46) (width 1.5) (layer F.Cu) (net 18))
 (segment (start 20.3708 -12.2682) (end 20.3708 -22.4536) (width 1.5) (layer F.Cu) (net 17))
 (segment (start 20.3708 -22.4536) (end 29.04 -31.1228) (width 1.5) (layer F.Cu) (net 17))
 (segment (start 29.04 -31.1228) (end 29.04 -37.46) (width 1.5) (layer F.Cu) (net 17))
 (segment (start 14.08 -5.9774) (end 20.3708 -12.2682) (width 1.5) (layer F.Cu) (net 17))
 (segment (start 14.08 7.46) (end 14.08 -5.9774) (width 1.5) (layer F.Cu) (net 17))
 (segment (start 41.8 -5.4694) (end 38.1254 -9.144) (width 1.5) (layer F.Cu) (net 16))
 (segment (start 40.894 -20.5994) (end 56.7944 -20.5994) (width 1.5) (layer F.Cu) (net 16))
 (segment (start 66.96 -10.4338) (end 66.96 7.46) (width 1.5) (layer F.Cu) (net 16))
 (segment (start 41.8 7.46) (end 41.8 -5.4694) (width 1.5) (layer F.Cu) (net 16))
 (segment (start 38.1254 -9.144) (end 38.1254 -17.8308) (width 1.5) (layer F.Cu) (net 16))
 (segment (start 38.1254 -17.8308) (end 40.894 -20.5994) (width 1.5) (layer F.Cu) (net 16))
 (segment (start 56.7944 -20.5994) (end 66.96 -10.4338) (width 1.5) (layer F.Cu) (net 16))
 (segment (start 45.76 7.46) (end 45.76 -7.3514) (width 1.5) (layer F.Cu) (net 15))
 (segment (start 45.76 -7.3514) (end 43 -10.1114) (width 1.5) (layer F.Cu) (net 15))
 (segment (start 43 -13.3118) (end 42.9768 -13.335) (width 1) (layer F.Cu) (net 15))
 (segment (start 43 -10.1114) (end 43 -13.3118) (width 1) (layer F.Cu) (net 15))
 (segment (start 25 -16.6814) (end 25.019 -16.6624) (width 1) (layer F.Cu) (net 6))
 (segment (start 25 -19.0056) (end 25 -16.6814) (width 1) (layer F.Cu) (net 6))
 (segment (start 25 -23.7554) (end 25 -19.0056) (width 1.5) (layer F.Cu) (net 6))
 (segment (start 36.96 -35.7154) (end 25 -23.7554) (width 1.5) (layer F.Cu) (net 6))
 (segment (start 36.96 -37.46) (end 36.96 -35.7154) (width 1.5) (layer F.Cu) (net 6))
 (segment (start 34 -17.7694) (end 34 -16.6984) (width 1) (layer F.Cu) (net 13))
 (segment (start 59.96 -37.46) (end 59.96 -25.6192) (width 1.5) (layer F.Cu) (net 13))
 (segment (start 34 -16.6984) (end 34.0106 -16.6878) (width 1) (layer F.Cu) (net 13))
 (segment (start 39.3192 -23.0886) (end 34 -17.7694) (width 1.5) (layer F.Cu) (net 13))
 (segment (start 59.96 -25.6192) (end 57.4294 -23.0886) (width 1.5) (layer F.Cu) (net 13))
 (segment (start 57.4294 -23.0886) (end 39.3192 -23.0886) (width 1.5) (layer F.Cu) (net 13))
 (segment (start 43 -16.6392) (end 43.0022 -16.637) (width 1) (layer F.Cu) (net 20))
 (segment (start 43 -17.9048) (end 43 -16.6392) (width 1) (layer F.Cu) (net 20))
 (segment (start 59.04 -0.1166) (end 47.2186 -11.938) (width 1.5) (layer F.Cu) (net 20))
 (segment (start 47.2186 -11.938) (end 47.2186 -17.2212) (width 1.5) (layer F.Cu) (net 20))
 (segment (start 47.2186 -17.2212) (end 45.8724 -18.5674) (width 1.5) (layer F.Cu) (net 20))
 (segment (start 43.6626 -18.5674) (end 43 -17.9048) (width 1.5) (layer F.Cu) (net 20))
 (segment (start 45.8724 -18.5674) (end 43.6626 -18.5674) (width 1.5) (layer F.Cu) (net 20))
 (segment (start 59.04 7.46) (end 59.04 -0.1166) (width 1.5) (layer F.Cu) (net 20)))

